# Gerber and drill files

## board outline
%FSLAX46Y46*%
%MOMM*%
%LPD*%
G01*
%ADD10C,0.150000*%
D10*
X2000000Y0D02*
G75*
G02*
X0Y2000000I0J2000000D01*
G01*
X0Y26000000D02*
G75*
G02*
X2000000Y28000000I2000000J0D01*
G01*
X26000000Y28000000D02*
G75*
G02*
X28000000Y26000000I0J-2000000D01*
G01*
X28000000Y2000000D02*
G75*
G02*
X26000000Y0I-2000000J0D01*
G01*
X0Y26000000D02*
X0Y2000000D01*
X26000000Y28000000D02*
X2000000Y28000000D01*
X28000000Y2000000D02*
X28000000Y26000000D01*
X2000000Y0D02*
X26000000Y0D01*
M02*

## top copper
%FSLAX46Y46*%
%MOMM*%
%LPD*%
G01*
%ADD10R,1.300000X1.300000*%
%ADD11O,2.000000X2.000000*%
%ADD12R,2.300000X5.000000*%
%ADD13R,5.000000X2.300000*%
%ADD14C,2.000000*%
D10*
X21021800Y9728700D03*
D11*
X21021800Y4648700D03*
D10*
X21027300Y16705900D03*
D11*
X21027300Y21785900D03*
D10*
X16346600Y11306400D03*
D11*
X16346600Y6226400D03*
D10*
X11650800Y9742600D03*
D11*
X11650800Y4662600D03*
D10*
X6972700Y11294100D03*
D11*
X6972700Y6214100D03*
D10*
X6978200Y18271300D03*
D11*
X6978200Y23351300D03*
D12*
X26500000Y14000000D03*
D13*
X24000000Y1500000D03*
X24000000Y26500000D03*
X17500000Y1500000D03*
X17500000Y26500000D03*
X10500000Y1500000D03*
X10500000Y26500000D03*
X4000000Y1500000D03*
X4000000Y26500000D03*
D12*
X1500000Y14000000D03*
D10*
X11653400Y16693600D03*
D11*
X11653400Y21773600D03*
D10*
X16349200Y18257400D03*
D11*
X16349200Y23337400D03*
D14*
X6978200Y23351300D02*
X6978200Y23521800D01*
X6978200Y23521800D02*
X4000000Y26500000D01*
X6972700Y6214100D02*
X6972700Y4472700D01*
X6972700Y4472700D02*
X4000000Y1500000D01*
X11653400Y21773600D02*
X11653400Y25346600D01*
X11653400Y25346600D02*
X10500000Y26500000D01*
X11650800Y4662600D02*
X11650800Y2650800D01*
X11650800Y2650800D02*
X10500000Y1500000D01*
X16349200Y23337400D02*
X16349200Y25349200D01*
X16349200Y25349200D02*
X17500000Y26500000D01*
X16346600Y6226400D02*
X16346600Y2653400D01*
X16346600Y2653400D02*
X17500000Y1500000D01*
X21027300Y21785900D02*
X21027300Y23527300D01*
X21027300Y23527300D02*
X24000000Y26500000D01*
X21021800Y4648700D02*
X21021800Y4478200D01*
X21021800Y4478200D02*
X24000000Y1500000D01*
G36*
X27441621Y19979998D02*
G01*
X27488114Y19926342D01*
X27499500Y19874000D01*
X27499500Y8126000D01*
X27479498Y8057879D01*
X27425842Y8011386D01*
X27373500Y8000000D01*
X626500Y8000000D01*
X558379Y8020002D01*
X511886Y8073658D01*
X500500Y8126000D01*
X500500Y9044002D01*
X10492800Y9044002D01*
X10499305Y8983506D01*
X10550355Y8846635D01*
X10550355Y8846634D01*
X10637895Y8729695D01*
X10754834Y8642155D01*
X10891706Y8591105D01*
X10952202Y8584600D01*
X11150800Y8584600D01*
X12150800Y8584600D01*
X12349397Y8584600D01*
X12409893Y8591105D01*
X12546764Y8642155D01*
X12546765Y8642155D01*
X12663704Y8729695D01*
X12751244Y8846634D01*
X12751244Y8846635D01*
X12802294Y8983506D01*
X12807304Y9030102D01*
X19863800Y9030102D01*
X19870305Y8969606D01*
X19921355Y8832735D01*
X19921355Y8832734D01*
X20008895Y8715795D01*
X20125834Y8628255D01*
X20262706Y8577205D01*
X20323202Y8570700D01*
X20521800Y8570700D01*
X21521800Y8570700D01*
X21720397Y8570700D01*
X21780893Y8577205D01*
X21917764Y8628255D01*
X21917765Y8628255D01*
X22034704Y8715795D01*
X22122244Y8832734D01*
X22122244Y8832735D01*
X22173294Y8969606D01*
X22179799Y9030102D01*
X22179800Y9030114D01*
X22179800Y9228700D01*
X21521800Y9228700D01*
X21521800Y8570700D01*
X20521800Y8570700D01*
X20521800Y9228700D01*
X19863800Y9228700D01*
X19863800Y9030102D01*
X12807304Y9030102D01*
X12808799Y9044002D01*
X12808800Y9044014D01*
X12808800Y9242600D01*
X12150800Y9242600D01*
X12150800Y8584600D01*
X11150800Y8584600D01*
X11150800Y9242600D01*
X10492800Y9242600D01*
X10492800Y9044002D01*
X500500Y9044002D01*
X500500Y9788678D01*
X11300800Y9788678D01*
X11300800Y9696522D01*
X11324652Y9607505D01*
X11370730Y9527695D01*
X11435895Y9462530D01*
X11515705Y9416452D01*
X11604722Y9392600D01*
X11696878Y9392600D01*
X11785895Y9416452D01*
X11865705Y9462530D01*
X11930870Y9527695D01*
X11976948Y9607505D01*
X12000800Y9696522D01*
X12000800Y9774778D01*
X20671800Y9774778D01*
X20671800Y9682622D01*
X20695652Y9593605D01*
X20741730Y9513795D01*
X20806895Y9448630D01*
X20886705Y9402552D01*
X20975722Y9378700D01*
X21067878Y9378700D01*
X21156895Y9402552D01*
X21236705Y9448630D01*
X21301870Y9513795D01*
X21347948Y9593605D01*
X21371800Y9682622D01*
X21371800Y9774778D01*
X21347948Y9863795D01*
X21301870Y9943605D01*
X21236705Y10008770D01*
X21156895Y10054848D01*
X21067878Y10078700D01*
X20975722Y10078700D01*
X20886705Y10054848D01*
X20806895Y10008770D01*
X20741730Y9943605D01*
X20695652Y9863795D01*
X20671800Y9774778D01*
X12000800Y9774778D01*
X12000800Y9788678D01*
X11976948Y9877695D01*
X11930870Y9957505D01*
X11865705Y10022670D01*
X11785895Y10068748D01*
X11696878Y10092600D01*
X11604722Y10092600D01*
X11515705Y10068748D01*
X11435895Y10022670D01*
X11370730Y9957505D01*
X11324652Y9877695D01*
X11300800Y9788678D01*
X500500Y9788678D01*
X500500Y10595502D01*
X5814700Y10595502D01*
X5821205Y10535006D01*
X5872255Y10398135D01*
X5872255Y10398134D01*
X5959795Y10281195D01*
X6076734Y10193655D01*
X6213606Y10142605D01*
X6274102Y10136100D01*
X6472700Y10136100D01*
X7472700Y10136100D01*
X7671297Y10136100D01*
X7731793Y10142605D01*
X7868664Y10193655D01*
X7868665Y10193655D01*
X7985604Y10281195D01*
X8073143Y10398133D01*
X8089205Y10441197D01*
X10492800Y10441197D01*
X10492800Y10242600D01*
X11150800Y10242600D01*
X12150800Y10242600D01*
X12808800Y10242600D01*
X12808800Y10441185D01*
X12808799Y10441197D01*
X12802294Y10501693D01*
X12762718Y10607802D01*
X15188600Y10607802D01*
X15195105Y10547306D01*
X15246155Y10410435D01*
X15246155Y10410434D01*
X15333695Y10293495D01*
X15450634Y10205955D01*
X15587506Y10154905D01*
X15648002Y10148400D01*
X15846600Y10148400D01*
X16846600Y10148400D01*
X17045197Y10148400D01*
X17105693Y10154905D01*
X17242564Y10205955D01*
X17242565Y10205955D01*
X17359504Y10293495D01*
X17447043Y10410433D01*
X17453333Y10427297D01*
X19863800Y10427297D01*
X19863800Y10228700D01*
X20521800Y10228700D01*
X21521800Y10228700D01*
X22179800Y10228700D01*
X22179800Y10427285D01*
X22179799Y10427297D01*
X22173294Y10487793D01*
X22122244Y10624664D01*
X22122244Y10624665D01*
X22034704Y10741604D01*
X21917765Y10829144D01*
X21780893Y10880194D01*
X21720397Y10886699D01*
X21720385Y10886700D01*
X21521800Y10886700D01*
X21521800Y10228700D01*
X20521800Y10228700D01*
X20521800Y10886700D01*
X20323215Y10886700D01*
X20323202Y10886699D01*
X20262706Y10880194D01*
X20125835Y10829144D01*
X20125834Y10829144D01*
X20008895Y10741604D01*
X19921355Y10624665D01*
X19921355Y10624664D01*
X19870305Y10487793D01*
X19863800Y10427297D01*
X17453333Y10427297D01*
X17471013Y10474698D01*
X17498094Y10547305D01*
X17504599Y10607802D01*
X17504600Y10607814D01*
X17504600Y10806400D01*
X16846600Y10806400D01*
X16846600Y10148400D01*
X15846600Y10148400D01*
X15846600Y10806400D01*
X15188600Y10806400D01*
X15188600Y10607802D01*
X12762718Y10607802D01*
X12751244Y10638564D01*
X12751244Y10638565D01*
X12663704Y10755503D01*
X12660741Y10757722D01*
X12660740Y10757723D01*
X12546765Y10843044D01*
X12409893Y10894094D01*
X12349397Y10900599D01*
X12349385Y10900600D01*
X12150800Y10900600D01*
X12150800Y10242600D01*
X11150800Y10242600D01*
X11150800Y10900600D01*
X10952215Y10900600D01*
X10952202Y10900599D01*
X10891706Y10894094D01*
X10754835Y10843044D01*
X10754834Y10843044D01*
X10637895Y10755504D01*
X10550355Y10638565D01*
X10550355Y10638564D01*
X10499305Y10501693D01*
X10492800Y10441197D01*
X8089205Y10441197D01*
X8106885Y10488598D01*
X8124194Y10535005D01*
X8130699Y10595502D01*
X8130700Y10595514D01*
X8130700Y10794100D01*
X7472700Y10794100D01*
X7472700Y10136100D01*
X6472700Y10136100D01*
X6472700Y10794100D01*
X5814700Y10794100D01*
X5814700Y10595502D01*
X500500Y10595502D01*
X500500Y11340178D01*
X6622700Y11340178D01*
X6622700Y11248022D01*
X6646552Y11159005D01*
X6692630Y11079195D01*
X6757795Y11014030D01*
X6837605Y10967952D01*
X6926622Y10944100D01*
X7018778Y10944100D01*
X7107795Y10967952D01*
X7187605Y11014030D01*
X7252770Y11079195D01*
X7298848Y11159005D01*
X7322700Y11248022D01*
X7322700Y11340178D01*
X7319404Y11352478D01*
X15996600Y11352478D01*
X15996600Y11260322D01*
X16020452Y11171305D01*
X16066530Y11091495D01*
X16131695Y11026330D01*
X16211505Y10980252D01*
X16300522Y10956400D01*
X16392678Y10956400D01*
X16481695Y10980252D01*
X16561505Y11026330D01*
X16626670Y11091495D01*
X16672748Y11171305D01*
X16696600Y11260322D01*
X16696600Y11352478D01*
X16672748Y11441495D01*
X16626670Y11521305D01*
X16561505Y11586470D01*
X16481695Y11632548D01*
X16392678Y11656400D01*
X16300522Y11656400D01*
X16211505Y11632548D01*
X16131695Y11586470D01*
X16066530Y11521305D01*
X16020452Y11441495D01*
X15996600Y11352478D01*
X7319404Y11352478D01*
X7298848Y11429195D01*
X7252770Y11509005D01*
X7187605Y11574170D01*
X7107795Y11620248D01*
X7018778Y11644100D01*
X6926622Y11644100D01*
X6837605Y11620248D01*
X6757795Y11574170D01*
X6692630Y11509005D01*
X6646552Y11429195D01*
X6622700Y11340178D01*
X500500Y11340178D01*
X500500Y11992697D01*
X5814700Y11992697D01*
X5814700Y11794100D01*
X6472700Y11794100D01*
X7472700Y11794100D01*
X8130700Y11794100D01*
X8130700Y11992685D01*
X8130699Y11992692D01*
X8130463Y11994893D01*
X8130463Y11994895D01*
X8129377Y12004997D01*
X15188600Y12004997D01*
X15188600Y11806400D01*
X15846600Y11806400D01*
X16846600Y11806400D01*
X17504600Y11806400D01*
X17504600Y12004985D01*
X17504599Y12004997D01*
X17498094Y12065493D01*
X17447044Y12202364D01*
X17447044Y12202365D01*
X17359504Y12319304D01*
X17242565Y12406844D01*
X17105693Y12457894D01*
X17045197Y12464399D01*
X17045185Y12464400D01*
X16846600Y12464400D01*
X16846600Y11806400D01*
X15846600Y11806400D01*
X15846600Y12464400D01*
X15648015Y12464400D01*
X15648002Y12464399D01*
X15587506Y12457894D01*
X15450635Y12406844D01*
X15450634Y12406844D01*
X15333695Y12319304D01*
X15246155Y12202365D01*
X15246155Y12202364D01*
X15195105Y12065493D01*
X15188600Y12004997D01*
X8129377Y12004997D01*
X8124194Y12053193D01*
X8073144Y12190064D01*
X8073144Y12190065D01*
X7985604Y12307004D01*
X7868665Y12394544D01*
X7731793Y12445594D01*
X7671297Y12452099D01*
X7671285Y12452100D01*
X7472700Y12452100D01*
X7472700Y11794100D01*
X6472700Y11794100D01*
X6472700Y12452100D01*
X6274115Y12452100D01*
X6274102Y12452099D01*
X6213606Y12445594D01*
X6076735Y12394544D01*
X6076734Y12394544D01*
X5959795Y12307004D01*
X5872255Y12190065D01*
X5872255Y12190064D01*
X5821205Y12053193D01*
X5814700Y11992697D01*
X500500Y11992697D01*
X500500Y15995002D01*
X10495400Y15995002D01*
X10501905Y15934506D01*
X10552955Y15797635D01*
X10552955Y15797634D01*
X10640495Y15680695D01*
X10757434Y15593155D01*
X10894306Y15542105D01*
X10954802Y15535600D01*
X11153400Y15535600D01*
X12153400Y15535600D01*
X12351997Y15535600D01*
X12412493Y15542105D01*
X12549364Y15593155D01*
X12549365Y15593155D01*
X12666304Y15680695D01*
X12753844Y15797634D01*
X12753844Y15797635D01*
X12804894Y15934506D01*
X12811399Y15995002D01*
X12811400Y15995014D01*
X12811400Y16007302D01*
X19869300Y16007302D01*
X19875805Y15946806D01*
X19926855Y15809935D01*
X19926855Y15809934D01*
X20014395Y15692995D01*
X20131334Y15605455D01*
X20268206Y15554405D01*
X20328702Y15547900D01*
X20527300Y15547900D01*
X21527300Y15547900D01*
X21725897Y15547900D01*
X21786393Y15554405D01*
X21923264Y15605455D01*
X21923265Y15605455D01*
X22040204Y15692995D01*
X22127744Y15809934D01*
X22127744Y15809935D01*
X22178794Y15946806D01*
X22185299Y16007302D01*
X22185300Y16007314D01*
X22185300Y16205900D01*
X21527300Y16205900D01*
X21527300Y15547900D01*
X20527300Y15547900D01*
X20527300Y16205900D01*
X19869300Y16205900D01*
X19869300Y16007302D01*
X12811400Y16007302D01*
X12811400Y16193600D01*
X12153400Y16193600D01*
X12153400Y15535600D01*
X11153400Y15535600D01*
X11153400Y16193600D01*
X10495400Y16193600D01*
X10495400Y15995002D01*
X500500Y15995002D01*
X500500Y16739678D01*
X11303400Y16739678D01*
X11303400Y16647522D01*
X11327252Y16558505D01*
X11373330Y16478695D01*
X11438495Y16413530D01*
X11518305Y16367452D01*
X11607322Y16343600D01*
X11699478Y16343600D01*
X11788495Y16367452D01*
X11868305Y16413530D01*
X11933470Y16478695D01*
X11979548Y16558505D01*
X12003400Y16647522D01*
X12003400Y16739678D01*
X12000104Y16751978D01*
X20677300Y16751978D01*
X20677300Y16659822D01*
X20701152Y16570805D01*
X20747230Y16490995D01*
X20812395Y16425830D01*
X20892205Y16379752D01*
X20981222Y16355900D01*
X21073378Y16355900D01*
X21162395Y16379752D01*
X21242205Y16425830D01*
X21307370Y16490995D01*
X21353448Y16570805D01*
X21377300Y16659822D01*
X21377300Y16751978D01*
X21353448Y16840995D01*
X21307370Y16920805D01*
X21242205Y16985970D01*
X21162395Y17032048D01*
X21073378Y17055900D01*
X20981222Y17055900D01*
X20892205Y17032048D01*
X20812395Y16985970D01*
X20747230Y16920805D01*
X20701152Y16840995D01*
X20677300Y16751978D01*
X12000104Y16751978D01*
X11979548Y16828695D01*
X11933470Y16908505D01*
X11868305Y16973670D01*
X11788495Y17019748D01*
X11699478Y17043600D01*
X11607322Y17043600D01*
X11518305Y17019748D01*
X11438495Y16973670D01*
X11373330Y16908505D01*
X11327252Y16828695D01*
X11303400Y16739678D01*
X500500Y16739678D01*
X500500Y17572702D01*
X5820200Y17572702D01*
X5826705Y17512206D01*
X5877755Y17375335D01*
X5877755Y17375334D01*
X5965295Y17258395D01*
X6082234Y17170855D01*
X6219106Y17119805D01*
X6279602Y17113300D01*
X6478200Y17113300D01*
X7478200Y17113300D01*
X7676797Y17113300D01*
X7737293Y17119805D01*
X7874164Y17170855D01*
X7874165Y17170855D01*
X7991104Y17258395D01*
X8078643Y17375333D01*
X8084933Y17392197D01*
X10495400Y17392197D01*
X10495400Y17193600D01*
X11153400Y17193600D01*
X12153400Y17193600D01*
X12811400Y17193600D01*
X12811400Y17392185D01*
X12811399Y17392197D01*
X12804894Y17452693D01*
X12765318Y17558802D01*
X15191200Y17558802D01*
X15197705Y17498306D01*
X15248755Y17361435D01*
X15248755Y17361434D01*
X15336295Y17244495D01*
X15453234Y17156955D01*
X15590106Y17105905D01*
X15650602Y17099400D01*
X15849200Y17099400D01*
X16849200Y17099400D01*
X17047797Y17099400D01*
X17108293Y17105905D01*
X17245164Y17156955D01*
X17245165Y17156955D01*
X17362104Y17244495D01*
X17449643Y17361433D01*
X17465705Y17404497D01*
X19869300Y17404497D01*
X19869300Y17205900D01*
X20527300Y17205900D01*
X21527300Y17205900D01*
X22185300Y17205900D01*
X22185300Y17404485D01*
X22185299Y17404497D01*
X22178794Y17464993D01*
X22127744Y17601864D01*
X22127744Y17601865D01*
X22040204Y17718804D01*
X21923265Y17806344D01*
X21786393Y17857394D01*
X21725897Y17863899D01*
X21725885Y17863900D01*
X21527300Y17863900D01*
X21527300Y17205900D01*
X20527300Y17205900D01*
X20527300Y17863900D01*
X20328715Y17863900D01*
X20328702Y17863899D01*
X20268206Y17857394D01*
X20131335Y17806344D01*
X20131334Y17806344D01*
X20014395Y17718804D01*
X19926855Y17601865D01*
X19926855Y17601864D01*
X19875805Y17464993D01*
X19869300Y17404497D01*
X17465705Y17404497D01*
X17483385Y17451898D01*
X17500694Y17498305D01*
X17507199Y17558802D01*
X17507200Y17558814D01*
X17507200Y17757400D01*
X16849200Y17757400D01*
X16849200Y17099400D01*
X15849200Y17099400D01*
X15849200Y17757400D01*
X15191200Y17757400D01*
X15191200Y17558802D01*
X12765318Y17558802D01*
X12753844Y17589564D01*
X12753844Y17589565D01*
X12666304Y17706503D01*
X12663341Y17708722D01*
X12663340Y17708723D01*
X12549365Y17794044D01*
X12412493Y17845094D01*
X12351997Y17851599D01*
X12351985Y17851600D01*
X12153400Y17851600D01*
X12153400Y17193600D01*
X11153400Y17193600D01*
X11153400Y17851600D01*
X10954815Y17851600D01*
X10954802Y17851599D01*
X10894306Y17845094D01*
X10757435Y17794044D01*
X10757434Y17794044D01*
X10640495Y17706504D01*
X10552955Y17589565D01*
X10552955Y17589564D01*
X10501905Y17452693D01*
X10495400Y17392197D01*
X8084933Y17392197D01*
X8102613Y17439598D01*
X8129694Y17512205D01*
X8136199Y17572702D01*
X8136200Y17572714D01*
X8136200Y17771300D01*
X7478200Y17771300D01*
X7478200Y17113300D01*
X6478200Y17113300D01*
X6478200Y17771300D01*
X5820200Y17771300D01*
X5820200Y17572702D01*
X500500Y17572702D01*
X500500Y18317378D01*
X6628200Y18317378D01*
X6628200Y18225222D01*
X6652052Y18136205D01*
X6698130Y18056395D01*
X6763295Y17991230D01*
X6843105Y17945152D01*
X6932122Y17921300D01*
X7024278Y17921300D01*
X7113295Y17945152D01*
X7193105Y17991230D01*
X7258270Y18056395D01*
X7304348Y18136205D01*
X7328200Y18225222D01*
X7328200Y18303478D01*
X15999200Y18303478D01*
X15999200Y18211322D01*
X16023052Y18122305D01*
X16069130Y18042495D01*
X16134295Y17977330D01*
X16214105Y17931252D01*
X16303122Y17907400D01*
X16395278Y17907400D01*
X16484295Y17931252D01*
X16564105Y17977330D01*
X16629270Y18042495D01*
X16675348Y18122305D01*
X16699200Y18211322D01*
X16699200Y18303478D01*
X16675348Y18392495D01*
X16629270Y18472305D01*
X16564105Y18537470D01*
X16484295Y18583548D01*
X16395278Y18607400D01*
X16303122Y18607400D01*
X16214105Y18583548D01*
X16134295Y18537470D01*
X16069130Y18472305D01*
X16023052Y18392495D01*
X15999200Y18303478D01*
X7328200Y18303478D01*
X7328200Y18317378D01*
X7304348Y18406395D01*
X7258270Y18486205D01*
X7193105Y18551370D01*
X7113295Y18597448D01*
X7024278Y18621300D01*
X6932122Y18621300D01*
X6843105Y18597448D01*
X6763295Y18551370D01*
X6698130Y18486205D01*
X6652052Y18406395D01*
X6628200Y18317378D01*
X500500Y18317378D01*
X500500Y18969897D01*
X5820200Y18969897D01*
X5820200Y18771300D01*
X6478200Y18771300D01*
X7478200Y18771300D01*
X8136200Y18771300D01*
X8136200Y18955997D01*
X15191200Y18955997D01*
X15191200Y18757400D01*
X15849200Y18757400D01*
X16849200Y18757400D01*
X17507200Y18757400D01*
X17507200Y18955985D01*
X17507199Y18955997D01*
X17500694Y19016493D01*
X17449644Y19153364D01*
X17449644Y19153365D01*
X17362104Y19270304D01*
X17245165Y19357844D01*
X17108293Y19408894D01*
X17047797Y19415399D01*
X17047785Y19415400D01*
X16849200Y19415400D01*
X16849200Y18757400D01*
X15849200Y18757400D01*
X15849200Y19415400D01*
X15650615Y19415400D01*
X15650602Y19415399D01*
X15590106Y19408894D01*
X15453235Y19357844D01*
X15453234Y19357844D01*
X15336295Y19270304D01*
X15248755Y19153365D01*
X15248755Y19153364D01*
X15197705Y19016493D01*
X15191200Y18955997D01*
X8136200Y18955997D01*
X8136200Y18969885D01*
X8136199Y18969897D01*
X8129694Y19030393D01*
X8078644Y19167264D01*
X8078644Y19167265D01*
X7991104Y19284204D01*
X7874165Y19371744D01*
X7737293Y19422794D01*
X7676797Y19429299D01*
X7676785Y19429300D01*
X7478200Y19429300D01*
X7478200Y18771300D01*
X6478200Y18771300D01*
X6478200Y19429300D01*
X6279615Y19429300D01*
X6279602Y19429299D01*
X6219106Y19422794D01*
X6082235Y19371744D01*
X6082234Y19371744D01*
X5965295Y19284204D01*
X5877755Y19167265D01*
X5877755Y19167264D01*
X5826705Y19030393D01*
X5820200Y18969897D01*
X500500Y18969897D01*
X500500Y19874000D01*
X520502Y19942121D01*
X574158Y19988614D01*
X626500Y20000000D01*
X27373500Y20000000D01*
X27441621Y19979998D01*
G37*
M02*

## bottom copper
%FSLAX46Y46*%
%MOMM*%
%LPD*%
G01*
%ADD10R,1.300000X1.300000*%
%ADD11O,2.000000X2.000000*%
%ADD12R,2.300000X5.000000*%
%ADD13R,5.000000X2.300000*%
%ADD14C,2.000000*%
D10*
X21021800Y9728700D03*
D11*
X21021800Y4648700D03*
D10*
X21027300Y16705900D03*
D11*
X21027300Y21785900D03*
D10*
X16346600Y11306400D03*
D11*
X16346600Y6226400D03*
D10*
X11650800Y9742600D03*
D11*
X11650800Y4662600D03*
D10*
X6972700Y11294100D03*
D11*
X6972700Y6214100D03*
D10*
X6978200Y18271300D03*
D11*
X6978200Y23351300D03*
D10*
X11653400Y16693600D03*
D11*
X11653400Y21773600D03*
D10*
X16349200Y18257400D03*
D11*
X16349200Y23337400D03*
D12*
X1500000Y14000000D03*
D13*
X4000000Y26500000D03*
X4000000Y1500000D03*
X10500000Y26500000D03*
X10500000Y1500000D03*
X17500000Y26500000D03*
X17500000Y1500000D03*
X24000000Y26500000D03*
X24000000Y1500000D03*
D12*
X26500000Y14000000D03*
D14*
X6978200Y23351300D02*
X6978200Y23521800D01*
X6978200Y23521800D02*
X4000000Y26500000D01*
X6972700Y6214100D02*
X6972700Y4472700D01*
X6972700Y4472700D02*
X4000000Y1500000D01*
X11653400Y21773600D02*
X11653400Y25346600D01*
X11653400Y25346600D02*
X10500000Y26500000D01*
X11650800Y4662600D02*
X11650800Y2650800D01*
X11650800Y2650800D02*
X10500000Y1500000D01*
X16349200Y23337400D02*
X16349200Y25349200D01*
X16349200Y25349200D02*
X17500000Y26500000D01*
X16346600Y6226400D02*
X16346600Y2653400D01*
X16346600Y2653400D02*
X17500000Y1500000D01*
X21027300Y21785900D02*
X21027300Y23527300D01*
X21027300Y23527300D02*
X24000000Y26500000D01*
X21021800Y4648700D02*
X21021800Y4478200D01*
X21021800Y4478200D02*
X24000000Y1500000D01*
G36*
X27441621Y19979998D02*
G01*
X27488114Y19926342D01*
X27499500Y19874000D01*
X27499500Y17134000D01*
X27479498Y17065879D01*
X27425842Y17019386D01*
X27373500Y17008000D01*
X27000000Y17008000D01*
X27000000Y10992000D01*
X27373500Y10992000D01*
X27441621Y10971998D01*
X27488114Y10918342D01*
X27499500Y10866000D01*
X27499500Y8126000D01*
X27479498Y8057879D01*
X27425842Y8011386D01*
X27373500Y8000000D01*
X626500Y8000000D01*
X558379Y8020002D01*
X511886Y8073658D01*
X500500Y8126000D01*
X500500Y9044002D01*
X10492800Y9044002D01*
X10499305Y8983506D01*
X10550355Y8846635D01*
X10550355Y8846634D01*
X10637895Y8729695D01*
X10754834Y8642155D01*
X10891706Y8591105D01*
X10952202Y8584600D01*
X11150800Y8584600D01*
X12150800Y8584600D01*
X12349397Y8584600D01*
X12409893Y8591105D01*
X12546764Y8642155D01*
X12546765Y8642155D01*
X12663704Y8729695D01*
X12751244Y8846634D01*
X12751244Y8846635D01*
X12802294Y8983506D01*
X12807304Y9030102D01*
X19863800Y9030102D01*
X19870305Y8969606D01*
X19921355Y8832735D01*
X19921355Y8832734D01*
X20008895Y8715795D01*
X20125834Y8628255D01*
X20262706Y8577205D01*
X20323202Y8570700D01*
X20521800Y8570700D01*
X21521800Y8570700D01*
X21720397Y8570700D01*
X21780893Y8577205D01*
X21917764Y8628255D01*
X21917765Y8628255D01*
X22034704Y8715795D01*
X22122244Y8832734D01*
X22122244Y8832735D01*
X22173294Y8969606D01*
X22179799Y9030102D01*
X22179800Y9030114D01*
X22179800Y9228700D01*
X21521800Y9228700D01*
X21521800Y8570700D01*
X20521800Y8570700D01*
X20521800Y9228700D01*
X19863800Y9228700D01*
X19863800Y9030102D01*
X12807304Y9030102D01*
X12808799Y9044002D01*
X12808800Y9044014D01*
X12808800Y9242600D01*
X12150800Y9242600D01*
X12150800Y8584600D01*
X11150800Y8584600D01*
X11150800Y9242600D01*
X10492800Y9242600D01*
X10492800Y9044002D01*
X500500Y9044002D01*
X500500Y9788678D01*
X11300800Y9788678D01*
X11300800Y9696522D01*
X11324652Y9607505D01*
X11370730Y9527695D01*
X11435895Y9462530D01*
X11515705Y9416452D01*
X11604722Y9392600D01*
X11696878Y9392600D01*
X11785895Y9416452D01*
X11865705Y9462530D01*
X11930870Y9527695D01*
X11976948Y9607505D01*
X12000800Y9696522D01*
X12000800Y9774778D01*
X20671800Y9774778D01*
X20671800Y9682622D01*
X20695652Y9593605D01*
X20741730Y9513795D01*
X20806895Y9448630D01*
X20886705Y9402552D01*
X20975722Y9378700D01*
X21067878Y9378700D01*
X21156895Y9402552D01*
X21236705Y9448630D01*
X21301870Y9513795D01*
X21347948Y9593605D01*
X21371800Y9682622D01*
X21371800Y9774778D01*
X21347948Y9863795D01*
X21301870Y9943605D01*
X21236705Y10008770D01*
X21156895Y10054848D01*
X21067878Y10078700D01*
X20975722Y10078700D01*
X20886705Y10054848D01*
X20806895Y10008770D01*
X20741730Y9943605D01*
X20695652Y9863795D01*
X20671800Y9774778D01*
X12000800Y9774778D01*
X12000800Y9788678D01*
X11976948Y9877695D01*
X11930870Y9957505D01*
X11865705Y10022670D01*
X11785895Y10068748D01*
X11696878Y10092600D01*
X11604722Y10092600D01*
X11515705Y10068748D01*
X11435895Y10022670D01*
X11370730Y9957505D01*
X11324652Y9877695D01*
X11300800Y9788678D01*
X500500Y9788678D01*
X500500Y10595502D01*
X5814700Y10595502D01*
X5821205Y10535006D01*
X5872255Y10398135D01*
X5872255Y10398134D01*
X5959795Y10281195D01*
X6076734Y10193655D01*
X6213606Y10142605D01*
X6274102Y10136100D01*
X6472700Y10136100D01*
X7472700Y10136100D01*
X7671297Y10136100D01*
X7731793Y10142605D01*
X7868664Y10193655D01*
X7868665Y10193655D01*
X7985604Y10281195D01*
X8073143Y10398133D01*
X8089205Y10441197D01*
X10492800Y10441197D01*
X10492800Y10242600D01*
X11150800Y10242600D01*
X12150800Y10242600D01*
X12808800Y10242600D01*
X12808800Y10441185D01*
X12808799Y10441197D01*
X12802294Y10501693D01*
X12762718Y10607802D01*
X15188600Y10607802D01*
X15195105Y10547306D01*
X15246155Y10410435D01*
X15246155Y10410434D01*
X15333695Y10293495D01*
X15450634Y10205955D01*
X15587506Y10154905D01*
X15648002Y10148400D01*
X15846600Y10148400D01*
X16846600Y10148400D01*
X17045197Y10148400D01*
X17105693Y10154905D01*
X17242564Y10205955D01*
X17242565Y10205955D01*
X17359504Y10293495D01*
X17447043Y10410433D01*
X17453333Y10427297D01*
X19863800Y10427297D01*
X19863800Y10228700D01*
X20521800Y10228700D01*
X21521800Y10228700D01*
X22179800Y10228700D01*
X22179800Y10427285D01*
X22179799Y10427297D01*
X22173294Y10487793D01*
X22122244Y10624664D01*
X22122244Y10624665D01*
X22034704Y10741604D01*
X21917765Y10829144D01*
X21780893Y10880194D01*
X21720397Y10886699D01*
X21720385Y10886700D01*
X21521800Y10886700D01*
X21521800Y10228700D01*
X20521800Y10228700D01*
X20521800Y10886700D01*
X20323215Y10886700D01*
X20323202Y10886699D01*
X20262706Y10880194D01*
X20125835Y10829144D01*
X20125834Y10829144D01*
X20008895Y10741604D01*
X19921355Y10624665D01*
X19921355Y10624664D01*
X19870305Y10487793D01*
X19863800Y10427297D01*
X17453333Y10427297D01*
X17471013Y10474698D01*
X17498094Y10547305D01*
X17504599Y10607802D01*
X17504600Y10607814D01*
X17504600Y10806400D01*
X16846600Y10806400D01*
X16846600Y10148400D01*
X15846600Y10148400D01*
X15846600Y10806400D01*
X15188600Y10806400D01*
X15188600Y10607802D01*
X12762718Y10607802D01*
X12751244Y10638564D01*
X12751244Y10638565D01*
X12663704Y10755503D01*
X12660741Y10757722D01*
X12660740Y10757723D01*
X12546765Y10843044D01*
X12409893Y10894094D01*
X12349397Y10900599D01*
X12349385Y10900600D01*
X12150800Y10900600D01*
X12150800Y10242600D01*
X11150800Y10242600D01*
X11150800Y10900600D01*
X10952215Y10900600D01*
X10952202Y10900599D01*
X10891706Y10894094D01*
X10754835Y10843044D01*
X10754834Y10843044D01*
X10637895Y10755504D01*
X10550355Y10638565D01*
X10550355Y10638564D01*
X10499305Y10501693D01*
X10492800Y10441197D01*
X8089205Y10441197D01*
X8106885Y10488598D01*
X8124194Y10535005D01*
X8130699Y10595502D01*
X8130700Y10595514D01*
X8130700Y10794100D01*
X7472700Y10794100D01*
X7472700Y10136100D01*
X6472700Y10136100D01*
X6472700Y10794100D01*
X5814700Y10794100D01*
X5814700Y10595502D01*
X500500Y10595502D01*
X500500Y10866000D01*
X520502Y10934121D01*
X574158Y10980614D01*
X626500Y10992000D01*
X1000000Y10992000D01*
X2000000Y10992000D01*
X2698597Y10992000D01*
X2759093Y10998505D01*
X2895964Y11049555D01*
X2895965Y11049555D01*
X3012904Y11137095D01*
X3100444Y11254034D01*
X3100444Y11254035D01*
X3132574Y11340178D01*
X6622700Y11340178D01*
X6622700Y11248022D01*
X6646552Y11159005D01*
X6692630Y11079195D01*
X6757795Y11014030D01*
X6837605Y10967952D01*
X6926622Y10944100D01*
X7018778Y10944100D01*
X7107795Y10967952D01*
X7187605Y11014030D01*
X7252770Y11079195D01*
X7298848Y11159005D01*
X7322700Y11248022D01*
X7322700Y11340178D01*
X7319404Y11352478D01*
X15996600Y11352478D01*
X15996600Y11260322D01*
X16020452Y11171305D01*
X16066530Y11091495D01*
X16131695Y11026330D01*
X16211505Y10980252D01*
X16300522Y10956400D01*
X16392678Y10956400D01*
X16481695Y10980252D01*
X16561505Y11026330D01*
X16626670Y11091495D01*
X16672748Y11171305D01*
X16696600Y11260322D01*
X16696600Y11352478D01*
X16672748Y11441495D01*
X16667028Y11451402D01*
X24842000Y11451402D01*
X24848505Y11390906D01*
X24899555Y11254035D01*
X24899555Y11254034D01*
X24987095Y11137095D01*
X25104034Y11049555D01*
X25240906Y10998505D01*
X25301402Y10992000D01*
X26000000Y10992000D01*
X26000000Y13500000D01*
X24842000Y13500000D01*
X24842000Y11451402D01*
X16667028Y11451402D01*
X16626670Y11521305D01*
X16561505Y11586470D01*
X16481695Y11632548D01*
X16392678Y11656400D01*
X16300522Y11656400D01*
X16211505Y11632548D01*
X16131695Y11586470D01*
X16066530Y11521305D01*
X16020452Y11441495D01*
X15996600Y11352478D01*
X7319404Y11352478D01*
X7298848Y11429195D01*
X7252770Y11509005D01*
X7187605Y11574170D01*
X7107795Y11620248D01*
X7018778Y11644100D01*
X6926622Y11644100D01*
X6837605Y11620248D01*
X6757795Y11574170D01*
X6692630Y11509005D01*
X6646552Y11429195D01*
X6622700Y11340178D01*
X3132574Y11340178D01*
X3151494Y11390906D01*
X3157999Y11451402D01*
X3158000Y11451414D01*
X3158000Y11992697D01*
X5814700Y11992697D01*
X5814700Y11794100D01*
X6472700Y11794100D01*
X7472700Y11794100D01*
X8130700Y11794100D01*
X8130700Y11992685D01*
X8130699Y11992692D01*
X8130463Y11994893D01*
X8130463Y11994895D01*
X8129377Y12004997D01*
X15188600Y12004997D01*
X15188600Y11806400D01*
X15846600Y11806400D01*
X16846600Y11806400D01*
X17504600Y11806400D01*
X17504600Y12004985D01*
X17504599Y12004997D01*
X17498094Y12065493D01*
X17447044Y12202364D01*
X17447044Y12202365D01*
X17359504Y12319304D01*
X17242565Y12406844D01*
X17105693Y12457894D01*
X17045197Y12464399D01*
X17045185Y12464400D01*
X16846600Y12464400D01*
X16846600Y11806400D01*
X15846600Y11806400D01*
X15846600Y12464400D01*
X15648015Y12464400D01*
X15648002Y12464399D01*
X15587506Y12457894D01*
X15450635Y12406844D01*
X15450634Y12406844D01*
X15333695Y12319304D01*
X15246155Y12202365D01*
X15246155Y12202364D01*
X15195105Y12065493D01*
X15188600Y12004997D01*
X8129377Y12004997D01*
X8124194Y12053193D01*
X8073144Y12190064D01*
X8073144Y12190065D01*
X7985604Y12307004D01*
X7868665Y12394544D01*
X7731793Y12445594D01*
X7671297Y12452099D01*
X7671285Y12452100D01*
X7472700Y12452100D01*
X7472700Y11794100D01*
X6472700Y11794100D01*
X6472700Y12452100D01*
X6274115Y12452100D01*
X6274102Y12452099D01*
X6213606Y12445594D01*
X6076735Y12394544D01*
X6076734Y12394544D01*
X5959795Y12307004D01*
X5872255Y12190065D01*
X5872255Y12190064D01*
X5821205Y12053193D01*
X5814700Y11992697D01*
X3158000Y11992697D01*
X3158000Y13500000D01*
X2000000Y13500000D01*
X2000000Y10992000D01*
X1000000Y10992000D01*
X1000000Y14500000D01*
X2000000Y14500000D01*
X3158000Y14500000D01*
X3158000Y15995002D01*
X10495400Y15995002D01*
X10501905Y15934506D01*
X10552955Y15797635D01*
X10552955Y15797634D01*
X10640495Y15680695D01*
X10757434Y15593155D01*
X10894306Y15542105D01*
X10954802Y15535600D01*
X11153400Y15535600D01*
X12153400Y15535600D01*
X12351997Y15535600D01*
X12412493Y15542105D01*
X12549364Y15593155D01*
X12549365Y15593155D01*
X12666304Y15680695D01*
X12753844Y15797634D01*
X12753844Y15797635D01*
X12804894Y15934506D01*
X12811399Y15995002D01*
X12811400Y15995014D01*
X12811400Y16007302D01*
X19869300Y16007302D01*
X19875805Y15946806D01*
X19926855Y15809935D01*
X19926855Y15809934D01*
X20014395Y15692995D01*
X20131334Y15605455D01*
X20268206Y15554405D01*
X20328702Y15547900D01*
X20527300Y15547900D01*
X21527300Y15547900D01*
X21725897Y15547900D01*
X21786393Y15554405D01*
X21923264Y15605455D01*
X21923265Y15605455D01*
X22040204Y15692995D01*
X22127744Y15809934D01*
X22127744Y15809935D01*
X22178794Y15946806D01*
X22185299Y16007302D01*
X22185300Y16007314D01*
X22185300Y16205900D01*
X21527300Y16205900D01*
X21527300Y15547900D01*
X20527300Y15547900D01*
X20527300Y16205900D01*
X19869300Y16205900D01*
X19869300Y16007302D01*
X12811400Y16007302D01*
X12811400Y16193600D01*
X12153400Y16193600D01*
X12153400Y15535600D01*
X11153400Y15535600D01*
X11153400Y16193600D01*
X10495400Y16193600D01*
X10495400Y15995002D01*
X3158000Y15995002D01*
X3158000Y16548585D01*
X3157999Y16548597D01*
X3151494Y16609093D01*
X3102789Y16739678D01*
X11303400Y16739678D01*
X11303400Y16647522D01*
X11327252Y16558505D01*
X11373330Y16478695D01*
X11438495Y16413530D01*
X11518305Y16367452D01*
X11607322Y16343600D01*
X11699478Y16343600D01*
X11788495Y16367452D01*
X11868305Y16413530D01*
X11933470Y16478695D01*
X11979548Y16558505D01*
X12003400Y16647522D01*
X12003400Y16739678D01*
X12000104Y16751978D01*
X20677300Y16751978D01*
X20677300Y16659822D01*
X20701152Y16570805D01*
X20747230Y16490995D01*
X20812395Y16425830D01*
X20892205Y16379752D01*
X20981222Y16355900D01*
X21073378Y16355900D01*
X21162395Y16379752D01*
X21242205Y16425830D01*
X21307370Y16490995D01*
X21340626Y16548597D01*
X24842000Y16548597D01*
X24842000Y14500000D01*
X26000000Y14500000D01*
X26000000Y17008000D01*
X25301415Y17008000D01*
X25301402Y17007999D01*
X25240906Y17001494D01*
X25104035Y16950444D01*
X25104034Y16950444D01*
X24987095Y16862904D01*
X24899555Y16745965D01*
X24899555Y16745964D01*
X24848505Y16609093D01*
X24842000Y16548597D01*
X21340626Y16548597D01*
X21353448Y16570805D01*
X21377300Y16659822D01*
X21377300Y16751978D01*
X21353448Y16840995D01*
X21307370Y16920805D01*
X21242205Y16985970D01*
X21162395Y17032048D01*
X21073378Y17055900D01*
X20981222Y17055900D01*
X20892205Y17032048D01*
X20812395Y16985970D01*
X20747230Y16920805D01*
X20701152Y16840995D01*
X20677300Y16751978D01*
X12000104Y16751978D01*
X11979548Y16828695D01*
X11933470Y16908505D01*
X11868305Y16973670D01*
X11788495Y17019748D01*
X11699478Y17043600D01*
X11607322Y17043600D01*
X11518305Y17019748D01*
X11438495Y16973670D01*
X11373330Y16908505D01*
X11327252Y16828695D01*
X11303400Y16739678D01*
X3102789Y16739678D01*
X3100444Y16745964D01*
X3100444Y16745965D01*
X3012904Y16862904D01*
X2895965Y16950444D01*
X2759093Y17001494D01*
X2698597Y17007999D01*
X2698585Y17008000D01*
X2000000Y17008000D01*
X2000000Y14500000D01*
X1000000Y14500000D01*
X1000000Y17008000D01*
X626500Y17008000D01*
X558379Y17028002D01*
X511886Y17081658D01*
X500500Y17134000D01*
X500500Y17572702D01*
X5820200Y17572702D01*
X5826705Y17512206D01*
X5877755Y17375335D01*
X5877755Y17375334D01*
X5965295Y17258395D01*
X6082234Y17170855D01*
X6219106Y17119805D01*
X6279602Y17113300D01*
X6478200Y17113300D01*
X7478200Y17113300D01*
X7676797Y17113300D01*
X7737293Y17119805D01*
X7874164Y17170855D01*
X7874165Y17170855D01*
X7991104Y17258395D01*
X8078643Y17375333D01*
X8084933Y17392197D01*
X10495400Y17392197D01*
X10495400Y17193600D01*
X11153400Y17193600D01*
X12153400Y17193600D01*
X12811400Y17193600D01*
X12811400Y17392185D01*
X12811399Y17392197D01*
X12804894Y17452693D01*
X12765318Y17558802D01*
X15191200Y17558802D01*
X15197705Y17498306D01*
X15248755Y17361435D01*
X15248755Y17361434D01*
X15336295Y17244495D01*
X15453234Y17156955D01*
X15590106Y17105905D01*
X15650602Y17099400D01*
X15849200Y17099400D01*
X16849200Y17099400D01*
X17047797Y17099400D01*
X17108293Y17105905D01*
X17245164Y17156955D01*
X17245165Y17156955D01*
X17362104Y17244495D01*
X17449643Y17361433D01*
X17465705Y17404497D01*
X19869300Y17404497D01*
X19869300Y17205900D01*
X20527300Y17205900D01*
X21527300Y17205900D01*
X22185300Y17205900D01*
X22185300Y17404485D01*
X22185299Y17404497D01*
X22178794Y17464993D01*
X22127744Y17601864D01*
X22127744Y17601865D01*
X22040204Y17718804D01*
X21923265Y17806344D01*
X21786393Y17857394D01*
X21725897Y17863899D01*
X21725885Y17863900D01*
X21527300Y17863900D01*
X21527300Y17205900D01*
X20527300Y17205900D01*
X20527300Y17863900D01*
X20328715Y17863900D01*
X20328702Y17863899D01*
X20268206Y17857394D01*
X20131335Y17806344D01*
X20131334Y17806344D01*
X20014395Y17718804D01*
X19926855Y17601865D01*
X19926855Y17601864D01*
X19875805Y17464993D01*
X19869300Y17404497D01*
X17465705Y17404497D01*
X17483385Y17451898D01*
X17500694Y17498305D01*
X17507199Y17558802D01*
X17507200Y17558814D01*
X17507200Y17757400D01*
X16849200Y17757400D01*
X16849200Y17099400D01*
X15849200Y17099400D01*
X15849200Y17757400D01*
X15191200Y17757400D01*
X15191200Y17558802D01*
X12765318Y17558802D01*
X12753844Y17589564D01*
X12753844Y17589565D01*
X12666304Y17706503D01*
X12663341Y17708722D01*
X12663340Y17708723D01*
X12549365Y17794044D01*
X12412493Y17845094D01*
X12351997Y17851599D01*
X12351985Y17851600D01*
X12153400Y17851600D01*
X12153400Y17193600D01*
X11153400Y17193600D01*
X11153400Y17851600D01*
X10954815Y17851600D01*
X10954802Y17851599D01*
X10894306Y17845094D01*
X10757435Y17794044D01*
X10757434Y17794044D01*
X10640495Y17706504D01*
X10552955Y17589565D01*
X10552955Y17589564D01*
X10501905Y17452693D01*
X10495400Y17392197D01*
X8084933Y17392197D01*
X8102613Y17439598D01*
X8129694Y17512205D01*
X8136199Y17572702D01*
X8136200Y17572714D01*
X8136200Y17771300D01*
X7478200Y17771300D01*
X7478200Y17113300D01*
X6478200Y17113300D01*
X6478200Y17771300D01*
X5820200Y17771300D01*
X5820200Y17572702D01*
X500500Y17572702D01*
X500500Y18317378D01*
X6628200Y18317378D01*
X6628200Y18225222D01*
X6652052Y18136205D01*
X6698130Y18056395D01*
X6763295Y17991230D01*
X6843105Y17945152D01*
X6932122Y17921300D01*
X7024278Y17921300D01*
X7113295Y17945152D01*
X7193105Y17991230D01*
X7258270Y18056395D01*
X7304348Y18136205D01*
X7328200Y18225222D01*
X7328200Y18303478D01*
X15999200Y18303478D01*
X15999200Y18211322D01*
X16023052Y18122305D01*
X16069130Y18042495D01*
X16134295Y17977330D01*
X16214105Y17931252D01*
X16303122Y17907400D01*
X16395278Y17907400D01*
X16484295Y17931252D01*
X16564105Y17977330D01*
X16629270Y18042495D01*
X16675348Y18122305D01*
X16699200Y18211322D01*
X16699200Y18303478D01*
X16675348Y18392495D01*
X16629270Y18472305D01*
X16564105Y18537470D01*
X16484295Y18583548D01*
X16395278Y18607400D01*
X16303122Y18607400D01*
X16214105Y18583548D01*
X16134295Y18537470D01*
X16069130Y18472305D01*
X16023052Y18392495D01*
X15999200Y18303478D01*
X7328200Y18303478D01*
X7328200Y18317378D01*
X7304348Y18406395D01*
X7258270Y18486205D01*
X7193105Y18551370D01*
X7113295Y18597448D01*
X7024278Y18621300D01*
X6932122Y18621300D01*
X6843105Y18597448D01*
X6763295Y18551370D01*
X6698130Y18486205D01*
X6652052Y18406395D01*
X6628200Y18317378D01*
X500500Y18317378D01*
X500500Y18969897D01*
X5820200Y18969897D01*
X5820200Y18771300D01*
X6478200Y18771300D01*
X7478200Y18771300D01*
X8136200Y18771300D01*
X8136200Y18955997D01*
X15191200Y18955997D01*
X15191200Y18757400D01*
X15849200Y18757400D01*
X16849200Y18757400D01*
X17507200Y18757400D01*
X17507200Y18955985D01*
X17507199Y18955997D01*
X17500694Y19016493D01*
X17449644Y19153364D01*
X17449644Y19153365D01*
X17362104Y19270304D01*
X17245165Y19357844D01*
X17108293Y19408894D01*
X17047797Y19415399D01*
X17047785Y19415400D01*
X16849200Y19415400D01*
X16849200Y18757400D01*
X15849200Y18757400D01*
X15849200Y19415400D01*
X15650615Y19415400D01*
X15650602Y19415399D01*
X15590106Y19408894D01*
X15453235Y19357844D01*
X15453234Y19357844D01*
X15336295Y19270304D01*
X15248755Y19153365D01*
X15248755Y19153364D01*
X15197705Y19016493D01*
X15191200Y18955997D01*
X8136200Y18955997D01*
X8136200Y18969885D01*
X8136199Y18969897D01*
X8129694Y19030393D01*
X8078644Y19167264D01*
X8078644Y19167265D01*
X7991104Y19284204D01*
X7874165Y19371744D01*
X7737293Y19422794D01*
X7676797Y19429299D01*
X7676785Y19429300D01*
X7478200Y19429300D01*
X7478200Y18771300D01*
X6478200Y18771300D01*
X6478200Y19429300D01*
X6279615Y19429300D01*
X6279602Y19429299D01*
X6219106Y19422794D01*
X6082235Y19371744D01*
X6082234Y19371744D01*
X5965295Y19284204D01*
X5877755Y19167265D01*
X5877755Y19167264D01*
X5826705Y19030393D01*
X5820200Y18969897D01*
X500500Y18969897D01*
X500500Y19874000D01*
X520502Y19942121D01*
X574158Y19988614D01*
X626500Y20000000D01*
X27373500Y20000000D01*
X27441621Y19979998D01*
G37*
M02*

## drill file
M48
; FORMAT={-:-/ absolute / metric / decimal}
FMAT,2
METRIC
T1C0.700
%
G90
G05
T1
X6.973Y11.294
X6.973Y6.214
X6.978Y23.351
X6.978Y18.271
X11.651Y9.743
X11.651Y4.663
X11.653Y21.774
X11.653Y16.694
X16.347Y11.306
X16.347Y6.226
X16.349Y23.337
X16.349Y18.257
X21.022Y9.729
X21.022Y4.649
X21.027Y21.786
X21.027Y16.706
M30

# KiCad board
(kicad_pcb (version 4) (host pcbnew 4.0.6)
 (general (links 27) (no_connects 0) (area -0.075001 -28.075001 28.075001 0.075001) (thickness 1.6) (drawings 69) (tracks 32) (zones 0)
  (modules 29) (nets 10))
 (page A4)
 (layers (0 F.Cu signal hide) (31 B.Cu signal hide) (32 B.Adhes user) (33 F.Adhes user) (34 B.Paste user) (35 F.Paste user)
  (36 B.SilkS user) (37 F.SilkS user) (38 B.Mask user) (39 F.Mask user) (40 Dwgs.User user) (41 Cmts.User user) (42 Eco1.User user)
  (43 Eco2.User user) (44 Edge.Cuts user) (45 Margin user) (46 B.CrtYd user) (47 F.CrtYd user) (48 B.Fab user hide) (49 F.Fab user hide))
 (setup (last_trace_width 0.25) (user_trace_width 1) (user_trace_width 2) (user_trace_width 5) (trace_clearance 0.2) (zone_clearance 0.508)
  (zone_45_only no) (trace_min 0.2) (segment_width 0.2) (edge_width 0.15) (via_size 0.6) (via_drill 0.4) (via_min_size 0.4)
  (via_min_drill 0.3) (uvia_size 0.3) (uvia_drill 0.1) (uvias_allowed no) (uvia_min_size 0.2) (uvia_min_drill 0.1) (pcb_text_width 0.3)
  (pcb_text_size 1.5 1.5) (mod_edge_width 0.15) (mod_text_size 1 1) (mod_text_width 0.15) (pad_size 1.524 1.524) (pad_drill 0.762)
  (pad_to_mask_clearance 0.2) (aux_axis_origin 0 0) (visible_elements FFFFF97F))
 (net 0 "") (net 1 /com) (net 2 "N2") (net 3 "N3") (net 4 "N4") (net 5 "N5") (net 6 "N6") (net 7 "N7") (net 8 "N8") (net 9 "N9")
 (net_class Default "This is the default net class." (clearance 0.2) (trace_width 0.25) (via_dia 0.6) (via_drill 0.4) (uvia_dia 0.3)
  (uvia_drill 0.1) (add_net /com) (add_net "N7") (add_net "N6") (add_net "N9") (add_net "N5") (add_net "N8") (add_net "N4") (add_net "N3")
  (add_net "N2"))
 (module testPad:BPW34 (layer B.Cu) (at 21.0218 -9.7287 270)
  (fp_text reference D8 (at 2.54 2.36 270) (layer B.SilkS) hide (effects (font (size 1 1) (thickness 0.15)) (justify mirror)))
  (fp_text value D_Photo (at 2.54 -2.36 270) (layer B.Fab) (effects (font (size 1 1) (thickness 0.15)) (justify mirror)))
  (pad 1 thru_hole rect (at 0 0 270) (size 1.3 1.3) (drill 0.7) (layers *.Cu *.Mask) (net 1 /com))
  (pad 2 thru_hole oval (at 5.08 0 270) (size 2 2) (drill 0.7) (layers *.Cu *.Mask) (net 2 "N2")))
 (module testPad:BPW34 (layer B.Cu) (at 21.0273 -16.7059 90)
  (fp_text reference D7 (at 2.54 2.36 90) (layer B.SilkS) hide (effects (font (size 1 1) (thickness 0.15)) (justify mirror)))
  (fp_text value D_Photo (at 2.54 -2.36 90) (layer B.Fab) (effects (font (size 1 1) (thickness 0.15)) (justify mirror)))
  (pad 1 thru_hole rect (at 0 0 90) (size 1.3 1.3) (drill 0.7) (layers *.Cu *.Mask) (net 1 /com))
  (pad 2 thru_hole oval (at 5.08 0 90) (size 2 2) (drill 0.7) (layers *.Cu *.Mask) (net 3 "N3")))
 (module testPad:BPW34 (layer B.Cu) (at 16.3466 -11.3064 270)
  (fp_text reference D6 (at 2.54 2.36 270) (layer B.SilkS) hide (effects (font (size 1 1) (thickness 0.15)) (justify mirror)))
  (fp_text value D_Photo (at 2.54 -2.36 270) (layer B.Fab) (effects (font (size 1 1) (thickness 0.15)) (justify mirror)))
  (pad 1 thru_hole rect (at 0 0 270) (size 1.3 1.3) (drill 0.7) (layers *.Cu *.Mask) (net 1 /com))
  (pad 2 thru_hole oval (at 5.08 0 270) (size 2 2) (drill 0.7) (layers *.Cu *.Mask) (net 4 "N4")))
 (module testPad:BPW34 (layer B.Cu) (at 11.6508 -9.7426 270)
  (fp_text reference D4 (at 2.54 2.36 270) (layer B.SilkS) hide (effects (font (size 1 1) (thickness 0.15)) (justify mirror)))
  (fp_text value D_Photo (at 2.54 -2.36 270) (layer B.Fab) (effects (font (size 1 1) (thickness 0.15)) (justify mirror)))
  (pad 1 thru_hole rect (at 0 0 270) (size 1.3 1.3) (drill 0.7) (layers *.Cu *.Mask) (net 1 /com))
  (pad 2 thru_hole oval (at 5.08 0 270) (size 2 2) (drill 0.7) (layers *.Cu *.Mask) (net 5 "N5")))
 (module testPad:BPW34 (layer B.Cu) (at 6.9727 -11.2941 270)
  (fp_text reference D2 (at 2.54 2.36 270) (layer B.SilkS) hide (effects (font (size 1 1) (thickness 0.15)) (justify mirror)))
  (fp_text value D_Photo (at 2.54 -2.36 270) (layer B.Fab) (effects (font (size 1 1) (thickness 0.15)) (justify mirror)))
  (pad 1 thru_hole rect (at 0 0 270) (size 1.3 1.3) (drill 0.7) (layers *.Cu *.Mask) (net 1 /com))
  (pad 2 thru_hole oval (at 5.08 0 270) (size 2 2) (drill 0.7) (layers *.Cu *.Mask) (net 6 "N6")))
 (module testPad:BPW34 (layer B.Cu) (at 6.9782 -18.2713 90)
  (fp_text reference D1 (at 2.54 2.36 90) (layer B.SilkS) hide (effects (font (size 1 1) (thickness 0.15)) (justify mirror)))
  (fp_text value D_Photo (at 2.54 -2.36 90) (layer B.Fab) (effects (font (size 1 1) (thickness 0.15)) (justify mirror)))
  (pad 1 thru_hole rect (at 0 0 90) (size 1.3 1.3) (drill 0.7) (layers *.Cu *.Mask) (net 1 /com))
  (pad 2 thru_hole oval (at 5.08 0 90) (size 2 2) (drill 0.7) (layers *.Cu *.Mask) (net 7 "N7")))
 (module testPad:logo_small (layer B.Cu) (at 14 -14 270)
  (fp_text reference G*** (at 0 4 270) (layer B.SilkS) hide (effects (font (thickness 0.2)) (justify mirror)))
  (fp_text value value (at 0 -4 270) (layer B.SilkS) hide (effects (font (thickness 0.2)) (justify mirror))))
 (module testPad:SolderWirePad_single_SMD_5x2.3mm (layer F.Cu) (at 26.5 -14 90)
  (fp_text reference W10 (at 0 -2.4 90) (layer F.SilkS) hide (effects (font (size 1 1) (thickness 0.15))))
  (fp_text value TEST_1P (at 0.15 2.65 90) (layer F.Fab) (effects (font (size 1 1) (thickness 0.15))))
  (pad 1 smd rect (at 0 0 90) (size 5 2.3) (layers F.Cu F.Paste F.Mask) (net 1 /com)))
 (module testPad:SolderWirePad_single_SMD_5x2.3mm (layer F.Cu) (at 24 -1.5)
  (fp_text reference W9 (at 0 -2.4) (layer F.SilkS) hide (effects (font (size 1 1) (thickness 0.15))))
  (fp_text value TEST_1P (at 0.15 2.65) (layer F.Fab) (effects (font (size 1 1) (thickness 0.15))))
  (pad 1 smd rect (at 0 0) (size 5 2.3) (layers F.Cu F.Paste F.Mask) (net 2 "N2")))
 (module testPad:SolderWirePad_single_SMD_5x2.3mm (layer F.Cu) (at 24 -26.5)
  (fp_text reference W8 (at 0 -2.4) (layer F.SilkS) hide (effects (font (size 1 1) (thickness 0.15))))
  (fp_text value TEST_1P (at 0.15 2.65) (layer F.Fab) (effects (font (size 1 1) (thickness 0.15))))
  (pad 1 smd rect (at 0 0) (size 5 2.3) (layers F.Cu F.Paste F.Mask) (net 3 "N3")))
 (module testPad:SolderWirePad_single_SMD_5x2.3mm (layer F.Cu) (at 17.5 -1.5)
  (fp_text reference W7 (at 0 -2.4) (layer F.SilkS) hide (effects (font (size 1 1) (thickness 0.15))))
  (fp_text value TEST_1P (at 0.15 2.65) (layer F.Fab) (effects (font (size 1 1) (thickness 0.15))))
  (pad 1 smd rect (at 0 0) (size 5 2.3) (layers F.Cu F.Paste F.Mask) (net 4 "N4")))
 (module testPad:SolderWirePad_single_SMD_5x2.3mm (layer F.Cu) (at 17.5 -26.5)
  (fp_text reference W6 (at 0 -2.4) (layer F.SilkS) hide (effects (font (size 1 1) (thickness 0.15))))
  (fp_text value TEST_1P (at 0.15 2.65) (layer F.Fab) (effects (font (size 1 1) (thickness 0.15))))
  (pad 1 smd rect (at 0 0) (size 5 2.3) (layers F.Cu F.Paste F.Mask) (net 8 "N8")))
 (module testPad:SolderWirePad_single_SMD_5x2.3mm (layer F.Cu) (at 10.5 -1.5)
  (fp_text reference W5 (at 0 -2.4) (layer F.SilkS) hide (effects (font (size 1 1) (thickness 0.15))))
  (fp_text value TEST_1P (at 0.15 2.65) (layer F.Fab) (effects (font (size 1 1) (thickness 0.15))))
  (pad 1 smd rect (at 0 0) (size 5 2.3) (layers F.Cu F.Paste F.Mask) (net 5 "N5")))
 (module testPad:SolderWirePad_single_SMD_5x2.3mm (layer F.Cu) (at 10.5 -26.5)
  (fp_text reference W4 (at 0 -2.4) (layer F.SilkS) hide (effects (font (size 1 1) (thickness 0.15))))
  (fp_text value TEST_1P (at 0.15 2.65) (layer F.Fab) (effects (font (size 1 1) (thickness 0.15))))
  (pad 1 smd rect (at 0 0) (size 5 2.3) (layers F.Cu F.Paste F.Mask) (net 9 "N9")))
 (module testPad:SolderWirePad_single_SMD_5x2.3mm (layer F.Cu) (at 4 -1.5)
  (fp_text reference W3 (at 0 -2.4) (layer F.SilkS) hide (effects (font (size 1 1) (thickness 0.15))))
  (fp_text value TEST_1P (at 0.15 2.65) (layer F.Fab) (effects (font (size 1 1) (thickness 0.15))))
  (pad 1 smd rect (at 0 0) (size 5 2.3) (layers F.Cu F.Paste F.Mask) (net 6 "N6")))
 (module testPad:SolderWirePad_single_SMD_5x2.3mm (layer F.Cu) (at 4 -26.5)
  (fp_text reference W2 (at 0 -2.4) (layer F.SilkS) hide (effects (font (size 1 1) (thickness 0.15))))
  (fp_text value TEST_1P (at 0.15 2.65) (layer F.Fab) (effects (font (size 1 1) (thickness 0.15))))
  (pad 1 smd rect (at 0 0) (size 5 2.3) (layers F.Cu F.Paste F.Mask) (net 7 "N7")))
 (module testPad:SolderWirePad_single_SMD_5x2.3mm (layer F.Cu) (at 1.5 -14 90)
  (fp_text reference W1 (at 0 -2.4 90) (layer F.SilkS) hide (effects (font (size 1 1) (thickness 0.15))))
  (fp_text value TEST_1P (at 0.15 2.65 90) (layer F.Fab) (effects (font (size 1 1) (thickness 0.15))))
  (pad 1 smd rect (at 0 0 90) (size 5 2.3) (layers F.Cu F.Paste F.Mask) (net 1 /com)))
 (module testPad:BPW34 (layer B.Cu) (at 11.6534 -16.6936 90)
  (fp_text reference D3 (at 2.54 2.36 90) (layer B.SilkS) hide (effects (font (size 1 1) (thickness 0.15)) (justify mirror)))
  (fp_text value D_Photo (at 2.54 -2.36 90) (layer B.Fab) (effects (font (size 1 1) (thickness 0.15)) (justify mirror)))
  (pad 1 thru_hole rect (at 0 0 90) (size 1.3 1.3) (drill 0.7) (layers *.Cu *.Mask) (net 1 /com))
  (pad 2 thru_hole oval (at 5.08 0 90) (size 2 2) (drill 0.7) (layers *.Cu *.Mask) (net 9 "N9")))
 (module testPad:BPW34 (layer B.Cu) (at 16.3492 -18.2574 90)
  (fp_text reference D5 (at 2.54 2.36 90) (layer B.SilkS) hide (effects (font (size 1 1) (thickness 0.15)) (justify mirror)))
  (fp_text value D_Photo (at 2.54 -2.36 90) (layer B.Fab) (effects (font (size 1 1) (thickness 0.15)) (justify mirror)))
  (pad 1 thru_hole rect (at 0 0 90) (size 1.3 1.3) (drill 0.7) (layers *.Cu *.Mask) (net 1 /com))
  (pad 2 thru_hole oval (at 5.08 0 90) (size 2 2) (drill 0.7) (layers *.Cu *.Mask) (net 8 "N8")))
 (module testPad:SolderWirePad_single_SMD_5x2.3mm (layer B.Cu) (at 1.5 -14 270)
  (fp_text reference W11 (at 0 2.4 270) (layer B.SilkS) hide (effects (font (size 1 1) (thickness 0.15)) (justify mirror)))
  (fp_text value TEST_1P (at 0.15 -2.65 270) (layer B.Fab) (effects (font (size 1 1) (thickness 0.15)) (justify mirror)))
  (pad 1 smd rect (at 0 0 270) (size 5 2.3) (layers B.Cu B.Paste B.Mask) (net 1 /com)))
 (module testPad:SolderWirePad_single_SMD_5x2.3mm (layer B.Cu) (at 4 -26.5)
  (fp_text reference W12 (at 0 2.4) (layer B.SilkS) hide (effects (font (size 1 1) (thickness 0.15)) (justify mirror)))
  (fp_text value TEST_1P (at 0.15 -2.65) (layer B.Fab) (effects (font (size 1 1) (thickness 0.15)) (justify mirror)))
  (pad 1 smd rect (at 0 0) (size 5 2.3) (layers B.Cu B.Paste B.Mask) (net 7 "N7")))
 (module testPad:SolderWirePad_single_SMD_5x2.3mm (layer B.Cu) (at 4 -1.5)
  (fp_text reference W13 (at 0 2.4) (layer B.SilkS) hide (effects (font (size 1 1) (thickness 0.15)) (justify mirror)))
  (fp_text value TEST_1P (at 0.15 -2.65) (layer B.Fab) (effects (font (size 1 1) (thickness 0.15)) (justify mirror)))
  (pad 1 smd rect (at 0 0) (size 5 2.3) (layers B.Cu B.Paste B.Mask) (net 6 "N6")))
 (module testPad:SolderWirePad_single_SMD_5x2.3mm (layer B.Cu) (at 10.5 -26.5)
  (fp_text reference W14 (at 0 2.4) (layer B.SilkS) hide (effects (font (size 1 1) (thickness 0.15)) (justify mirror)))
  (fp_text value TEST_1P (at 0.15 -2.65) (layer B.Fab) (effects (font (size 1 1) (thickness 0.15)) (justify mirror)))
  (pad 1 smd rect (at 0 0) (size 5 2.3) (layers B.Cu B.Paste B.Mask) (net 9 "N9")))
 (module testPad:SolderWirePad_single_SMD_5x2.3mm (layer B.Cu) (at 10.5 -1.5)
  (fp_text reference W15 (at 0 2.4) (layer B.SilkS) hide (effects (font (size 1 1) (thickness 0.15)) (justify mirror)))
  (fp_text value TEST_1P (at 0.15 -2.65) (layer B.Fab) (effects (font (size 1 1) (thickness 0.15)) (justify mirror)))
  (pad 1 smd rect (at 0 0) (size 5 2.3) (layers B.Cu B.Paste B.Mask) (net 5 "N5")))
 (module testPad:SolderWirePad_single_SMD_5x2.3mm (layer B.Cu) (at 17.5 -26.5)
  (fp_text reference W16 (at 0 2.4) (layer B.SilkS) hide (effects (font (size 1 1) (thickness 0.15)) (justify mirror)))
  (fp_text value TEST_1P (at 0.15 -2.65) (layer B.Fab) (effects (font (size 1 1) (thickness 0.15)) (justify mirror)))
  (pad 1 smd rect (at 0 0) (size 5 2.3) (layers B.Cu B.Paste B.Mask) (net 8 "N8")))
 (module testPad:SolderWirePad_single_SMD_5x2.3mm (layer B.Cu) (at 17.5 -1.5)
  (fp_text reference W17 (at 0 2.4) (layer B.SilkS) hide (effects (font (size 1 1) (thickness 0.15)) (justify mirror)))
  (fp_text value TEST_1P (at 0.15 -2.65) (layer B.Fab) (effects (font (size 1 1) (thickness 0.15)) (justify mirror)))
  (pad 1 smd rect (at 0 0) (size 5 2.3) (layers B.Cu B.Paste B.Mask) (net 4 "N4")))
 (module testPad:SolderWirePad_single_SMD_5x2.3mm (layer B.Cu) (at 24 -26.5)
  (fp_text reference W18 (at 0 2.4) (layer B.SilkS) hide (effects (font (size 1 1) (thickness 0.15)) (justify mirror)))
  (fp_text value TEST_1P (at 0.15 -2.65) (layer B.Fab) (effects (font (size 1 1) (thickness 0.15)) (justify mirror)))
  (pad 1 smd rect (at 0 0) (size 5 2.3) (layers B.Cu B.Paste B.Mask) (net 3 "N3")))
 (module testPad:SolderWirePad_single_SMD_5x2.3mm (layer B.Cu) (at 24 -1.5)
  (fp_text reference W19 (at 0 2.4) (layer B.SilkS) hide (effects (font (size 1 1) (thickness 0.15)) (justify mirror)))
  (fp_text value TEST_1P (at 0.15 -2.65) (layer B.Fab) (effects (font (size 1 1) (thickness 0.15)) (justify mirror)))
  (pad 1 smd rect (at 0 0) (size 5 2.3) (layers B.Cu B.Paste B.Mask) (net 2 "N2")))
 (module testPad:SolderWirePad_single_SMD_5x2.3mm (layer B.Cu) (at 26.5 -14 270)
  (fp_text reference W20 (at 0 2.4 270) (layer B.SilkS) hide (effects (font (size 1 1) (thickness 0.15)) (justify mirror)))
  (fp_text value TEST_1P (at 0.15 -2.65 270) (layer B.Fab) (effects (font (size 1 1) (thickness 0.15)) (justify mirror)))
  (pad 1 smd rect (at 0 0 270) (size 5 2.3) (layers B.Cu B.Paste B.Mask) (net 1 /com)))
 (gr_arc (start 2 -2) (end 2 0) (angle 90) (layer Edge.Cuts) (width 0.15))
 (gr_arc (start 2 -26) (end 0 -26) (angle 90) (layer Edge.Cuts) (width 0.15))
 (gr_arc (start 26 -26) (end 26 -28) (angle 90) (layer Edge.Cuts) (width 0.15))
 (gr_arc (start 26 -2) (end 28 -2) (angle 90) (layer Edge.Cuts) (width 0.15))
 (gr_line (start 0 -26) (end 0 -2) (layer Edge.Cuts) (width 0.15))
 (gr_line (start 26 -28) (end 2 -28) (layer Edge.Cuts) (width 0.15))
 (gr_line (start 28 -2) (end 28 -26) (layer Edge.Cuts) (width 0.15))
 (gr_line (start 2 0) (end 26 0) (layer Edge.Cuts) (width 0.15))
 (segment (start 6.9782 -23.3513) (end 6.9782 -23.5218) (width 2) (layer B.Cu) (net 7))
 (segment (start 6.9782 -23.5218) (end 4 -26.5) (width 2) (layer B.Cu) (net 7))
 (segment (start 6.9782 -23.3513) (end 6.9782 -23.5218) (width 2) (layer F.Cu) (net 7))
 (segment (start 6.9782 -23.5218) (end 4 -26.5) (width 2) (layer F.Cu) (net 7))
 (segment (start 6.9727 -6.2141) (end 6.9727 -4.4727) (width 2) (layer B.Cu) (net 6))
 (segment (start 6.9727 -4.4727) (end 4 -1.5) (width 2) (layer B.Cu) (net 6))
 (segment (start 6.9727 -6.2141) (end 6.9727 -4.4727) (width 2) (layer F.Cu) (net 6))
 (segment (start 6.9727 -4.4727) (end 4 -1.5) (width 2) (layer F.Cu) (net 6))
 (segment (start 11.6534 -21.7736) (end 11.6534 -25.3466) (width 2) (layer B.Cu) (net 9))
 (segment (start 11.6534 -25.3466) (end 10.5 -26.5) (width 2) (layer B.Cu) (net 9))
 (segment (start 11.6534 -21.7736) (end 11.6534 -25.3466) (width 2) (layer F.Cu) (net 9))
 (segment (start 11.6534 -25.3466) (end 10.5 -26.5) (width 2) (layer F.Cu) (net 9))
 (segment (start 11.6508 -4.6626) (end 11.6508 -2.6508) (width 2) (layer B.Cu) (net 5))
 (segment (start 11.6508 -2.6508) (end 10.5 -1.5) (width 2) (layer B.Cu) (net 5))
 (segment (start 11.6508 -4.6626) (end 11.6508 -2.6508) (width 2) (layer F.Cu) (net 5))
 (segment (start 11.6508 -2.6508) (end 10.5 -1.5) (width 2) (layer F.Cu) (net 5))
 (segment (start 16.3492 -23.3374) (end 16.3492 -25.3492) (width 2) (layer B.Cu) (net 8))
 (segment (start 16.3492 -25.3492) (end 17.5 -26.5) (width 2) (layer B.Cu) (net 8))
 (segment (start 16.3492 -23.3374) (end 16.3492 -25.3492) (width 2) (layer F.Cu) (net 8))
 (segment (start 16.3492 -25.3492) (end 17.5 -26.5) (width 2) (layer F.Cu) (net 8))
 (segment (start 16.3466 -6.2264) (end 16.3466 -2.6534) (width 2) (layer B.Cu) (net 4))
 (segment (start 16.3466 -2.6534) (end 17.5 -1.5) (width 2) (layer B.Cu) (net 4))
 (segment (start 16.3466 -6.2264) (end 16.3466 -2.6534) (width 2) (layer F.Cu) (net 4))
 (segment (start 16.3466 -2.6534) (end 17.5 -1.5) (width 2) (layer F.Cu) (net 4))
 (segment (start 21.0273 -21.7859) (end 21.0273 -23.5273) (width 2) (layer B.Cu) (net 3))
 (segment (start 21.0273 -23.5273) (end 24 -26.5) (width 2) (layer B.Cu) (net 3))
 (segment (start 21.0273 -21.7859) (end 21.0273 -23.5273) (width 2) (layer F.Cu) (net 3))
 (segment (start 21.0273 -23.5273) (end 24 -26.5) (width 2) (layer F.Cu) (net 3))
 (segment (start 21.0218 -4.6487) (end 21.0218 -4.4782) (width 2) (layer B.Cu) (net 2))
 (segment (start 21.0218 -4.4782) (end 24 -1.5) (width 2) (layer B.Cu) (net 2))
 (segment (start 21.0218 -4.6487) (end 21.0218 -4.4782) (width 2) (layer F.Cu) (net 2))
 (segment (start 21.0218 -4.4782) (end 24 -1.5) (width 2) (layer F.Cu) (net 2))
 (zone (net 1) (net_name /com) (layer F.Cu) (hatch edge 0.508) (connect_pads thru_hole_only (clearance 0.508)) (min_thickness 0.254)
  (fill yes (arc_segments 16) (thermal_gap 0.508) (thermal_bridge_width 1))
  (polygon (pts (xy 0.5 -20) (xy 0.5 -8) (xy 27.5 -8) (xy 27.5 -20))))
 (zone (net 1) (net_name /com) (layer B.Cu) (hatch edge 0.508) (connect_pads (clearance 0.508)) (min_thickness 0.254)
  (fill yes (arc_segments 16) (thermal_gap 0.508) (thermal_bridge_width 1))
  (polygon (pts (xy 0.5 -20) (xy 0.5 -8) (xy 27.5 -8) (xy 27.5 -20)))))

